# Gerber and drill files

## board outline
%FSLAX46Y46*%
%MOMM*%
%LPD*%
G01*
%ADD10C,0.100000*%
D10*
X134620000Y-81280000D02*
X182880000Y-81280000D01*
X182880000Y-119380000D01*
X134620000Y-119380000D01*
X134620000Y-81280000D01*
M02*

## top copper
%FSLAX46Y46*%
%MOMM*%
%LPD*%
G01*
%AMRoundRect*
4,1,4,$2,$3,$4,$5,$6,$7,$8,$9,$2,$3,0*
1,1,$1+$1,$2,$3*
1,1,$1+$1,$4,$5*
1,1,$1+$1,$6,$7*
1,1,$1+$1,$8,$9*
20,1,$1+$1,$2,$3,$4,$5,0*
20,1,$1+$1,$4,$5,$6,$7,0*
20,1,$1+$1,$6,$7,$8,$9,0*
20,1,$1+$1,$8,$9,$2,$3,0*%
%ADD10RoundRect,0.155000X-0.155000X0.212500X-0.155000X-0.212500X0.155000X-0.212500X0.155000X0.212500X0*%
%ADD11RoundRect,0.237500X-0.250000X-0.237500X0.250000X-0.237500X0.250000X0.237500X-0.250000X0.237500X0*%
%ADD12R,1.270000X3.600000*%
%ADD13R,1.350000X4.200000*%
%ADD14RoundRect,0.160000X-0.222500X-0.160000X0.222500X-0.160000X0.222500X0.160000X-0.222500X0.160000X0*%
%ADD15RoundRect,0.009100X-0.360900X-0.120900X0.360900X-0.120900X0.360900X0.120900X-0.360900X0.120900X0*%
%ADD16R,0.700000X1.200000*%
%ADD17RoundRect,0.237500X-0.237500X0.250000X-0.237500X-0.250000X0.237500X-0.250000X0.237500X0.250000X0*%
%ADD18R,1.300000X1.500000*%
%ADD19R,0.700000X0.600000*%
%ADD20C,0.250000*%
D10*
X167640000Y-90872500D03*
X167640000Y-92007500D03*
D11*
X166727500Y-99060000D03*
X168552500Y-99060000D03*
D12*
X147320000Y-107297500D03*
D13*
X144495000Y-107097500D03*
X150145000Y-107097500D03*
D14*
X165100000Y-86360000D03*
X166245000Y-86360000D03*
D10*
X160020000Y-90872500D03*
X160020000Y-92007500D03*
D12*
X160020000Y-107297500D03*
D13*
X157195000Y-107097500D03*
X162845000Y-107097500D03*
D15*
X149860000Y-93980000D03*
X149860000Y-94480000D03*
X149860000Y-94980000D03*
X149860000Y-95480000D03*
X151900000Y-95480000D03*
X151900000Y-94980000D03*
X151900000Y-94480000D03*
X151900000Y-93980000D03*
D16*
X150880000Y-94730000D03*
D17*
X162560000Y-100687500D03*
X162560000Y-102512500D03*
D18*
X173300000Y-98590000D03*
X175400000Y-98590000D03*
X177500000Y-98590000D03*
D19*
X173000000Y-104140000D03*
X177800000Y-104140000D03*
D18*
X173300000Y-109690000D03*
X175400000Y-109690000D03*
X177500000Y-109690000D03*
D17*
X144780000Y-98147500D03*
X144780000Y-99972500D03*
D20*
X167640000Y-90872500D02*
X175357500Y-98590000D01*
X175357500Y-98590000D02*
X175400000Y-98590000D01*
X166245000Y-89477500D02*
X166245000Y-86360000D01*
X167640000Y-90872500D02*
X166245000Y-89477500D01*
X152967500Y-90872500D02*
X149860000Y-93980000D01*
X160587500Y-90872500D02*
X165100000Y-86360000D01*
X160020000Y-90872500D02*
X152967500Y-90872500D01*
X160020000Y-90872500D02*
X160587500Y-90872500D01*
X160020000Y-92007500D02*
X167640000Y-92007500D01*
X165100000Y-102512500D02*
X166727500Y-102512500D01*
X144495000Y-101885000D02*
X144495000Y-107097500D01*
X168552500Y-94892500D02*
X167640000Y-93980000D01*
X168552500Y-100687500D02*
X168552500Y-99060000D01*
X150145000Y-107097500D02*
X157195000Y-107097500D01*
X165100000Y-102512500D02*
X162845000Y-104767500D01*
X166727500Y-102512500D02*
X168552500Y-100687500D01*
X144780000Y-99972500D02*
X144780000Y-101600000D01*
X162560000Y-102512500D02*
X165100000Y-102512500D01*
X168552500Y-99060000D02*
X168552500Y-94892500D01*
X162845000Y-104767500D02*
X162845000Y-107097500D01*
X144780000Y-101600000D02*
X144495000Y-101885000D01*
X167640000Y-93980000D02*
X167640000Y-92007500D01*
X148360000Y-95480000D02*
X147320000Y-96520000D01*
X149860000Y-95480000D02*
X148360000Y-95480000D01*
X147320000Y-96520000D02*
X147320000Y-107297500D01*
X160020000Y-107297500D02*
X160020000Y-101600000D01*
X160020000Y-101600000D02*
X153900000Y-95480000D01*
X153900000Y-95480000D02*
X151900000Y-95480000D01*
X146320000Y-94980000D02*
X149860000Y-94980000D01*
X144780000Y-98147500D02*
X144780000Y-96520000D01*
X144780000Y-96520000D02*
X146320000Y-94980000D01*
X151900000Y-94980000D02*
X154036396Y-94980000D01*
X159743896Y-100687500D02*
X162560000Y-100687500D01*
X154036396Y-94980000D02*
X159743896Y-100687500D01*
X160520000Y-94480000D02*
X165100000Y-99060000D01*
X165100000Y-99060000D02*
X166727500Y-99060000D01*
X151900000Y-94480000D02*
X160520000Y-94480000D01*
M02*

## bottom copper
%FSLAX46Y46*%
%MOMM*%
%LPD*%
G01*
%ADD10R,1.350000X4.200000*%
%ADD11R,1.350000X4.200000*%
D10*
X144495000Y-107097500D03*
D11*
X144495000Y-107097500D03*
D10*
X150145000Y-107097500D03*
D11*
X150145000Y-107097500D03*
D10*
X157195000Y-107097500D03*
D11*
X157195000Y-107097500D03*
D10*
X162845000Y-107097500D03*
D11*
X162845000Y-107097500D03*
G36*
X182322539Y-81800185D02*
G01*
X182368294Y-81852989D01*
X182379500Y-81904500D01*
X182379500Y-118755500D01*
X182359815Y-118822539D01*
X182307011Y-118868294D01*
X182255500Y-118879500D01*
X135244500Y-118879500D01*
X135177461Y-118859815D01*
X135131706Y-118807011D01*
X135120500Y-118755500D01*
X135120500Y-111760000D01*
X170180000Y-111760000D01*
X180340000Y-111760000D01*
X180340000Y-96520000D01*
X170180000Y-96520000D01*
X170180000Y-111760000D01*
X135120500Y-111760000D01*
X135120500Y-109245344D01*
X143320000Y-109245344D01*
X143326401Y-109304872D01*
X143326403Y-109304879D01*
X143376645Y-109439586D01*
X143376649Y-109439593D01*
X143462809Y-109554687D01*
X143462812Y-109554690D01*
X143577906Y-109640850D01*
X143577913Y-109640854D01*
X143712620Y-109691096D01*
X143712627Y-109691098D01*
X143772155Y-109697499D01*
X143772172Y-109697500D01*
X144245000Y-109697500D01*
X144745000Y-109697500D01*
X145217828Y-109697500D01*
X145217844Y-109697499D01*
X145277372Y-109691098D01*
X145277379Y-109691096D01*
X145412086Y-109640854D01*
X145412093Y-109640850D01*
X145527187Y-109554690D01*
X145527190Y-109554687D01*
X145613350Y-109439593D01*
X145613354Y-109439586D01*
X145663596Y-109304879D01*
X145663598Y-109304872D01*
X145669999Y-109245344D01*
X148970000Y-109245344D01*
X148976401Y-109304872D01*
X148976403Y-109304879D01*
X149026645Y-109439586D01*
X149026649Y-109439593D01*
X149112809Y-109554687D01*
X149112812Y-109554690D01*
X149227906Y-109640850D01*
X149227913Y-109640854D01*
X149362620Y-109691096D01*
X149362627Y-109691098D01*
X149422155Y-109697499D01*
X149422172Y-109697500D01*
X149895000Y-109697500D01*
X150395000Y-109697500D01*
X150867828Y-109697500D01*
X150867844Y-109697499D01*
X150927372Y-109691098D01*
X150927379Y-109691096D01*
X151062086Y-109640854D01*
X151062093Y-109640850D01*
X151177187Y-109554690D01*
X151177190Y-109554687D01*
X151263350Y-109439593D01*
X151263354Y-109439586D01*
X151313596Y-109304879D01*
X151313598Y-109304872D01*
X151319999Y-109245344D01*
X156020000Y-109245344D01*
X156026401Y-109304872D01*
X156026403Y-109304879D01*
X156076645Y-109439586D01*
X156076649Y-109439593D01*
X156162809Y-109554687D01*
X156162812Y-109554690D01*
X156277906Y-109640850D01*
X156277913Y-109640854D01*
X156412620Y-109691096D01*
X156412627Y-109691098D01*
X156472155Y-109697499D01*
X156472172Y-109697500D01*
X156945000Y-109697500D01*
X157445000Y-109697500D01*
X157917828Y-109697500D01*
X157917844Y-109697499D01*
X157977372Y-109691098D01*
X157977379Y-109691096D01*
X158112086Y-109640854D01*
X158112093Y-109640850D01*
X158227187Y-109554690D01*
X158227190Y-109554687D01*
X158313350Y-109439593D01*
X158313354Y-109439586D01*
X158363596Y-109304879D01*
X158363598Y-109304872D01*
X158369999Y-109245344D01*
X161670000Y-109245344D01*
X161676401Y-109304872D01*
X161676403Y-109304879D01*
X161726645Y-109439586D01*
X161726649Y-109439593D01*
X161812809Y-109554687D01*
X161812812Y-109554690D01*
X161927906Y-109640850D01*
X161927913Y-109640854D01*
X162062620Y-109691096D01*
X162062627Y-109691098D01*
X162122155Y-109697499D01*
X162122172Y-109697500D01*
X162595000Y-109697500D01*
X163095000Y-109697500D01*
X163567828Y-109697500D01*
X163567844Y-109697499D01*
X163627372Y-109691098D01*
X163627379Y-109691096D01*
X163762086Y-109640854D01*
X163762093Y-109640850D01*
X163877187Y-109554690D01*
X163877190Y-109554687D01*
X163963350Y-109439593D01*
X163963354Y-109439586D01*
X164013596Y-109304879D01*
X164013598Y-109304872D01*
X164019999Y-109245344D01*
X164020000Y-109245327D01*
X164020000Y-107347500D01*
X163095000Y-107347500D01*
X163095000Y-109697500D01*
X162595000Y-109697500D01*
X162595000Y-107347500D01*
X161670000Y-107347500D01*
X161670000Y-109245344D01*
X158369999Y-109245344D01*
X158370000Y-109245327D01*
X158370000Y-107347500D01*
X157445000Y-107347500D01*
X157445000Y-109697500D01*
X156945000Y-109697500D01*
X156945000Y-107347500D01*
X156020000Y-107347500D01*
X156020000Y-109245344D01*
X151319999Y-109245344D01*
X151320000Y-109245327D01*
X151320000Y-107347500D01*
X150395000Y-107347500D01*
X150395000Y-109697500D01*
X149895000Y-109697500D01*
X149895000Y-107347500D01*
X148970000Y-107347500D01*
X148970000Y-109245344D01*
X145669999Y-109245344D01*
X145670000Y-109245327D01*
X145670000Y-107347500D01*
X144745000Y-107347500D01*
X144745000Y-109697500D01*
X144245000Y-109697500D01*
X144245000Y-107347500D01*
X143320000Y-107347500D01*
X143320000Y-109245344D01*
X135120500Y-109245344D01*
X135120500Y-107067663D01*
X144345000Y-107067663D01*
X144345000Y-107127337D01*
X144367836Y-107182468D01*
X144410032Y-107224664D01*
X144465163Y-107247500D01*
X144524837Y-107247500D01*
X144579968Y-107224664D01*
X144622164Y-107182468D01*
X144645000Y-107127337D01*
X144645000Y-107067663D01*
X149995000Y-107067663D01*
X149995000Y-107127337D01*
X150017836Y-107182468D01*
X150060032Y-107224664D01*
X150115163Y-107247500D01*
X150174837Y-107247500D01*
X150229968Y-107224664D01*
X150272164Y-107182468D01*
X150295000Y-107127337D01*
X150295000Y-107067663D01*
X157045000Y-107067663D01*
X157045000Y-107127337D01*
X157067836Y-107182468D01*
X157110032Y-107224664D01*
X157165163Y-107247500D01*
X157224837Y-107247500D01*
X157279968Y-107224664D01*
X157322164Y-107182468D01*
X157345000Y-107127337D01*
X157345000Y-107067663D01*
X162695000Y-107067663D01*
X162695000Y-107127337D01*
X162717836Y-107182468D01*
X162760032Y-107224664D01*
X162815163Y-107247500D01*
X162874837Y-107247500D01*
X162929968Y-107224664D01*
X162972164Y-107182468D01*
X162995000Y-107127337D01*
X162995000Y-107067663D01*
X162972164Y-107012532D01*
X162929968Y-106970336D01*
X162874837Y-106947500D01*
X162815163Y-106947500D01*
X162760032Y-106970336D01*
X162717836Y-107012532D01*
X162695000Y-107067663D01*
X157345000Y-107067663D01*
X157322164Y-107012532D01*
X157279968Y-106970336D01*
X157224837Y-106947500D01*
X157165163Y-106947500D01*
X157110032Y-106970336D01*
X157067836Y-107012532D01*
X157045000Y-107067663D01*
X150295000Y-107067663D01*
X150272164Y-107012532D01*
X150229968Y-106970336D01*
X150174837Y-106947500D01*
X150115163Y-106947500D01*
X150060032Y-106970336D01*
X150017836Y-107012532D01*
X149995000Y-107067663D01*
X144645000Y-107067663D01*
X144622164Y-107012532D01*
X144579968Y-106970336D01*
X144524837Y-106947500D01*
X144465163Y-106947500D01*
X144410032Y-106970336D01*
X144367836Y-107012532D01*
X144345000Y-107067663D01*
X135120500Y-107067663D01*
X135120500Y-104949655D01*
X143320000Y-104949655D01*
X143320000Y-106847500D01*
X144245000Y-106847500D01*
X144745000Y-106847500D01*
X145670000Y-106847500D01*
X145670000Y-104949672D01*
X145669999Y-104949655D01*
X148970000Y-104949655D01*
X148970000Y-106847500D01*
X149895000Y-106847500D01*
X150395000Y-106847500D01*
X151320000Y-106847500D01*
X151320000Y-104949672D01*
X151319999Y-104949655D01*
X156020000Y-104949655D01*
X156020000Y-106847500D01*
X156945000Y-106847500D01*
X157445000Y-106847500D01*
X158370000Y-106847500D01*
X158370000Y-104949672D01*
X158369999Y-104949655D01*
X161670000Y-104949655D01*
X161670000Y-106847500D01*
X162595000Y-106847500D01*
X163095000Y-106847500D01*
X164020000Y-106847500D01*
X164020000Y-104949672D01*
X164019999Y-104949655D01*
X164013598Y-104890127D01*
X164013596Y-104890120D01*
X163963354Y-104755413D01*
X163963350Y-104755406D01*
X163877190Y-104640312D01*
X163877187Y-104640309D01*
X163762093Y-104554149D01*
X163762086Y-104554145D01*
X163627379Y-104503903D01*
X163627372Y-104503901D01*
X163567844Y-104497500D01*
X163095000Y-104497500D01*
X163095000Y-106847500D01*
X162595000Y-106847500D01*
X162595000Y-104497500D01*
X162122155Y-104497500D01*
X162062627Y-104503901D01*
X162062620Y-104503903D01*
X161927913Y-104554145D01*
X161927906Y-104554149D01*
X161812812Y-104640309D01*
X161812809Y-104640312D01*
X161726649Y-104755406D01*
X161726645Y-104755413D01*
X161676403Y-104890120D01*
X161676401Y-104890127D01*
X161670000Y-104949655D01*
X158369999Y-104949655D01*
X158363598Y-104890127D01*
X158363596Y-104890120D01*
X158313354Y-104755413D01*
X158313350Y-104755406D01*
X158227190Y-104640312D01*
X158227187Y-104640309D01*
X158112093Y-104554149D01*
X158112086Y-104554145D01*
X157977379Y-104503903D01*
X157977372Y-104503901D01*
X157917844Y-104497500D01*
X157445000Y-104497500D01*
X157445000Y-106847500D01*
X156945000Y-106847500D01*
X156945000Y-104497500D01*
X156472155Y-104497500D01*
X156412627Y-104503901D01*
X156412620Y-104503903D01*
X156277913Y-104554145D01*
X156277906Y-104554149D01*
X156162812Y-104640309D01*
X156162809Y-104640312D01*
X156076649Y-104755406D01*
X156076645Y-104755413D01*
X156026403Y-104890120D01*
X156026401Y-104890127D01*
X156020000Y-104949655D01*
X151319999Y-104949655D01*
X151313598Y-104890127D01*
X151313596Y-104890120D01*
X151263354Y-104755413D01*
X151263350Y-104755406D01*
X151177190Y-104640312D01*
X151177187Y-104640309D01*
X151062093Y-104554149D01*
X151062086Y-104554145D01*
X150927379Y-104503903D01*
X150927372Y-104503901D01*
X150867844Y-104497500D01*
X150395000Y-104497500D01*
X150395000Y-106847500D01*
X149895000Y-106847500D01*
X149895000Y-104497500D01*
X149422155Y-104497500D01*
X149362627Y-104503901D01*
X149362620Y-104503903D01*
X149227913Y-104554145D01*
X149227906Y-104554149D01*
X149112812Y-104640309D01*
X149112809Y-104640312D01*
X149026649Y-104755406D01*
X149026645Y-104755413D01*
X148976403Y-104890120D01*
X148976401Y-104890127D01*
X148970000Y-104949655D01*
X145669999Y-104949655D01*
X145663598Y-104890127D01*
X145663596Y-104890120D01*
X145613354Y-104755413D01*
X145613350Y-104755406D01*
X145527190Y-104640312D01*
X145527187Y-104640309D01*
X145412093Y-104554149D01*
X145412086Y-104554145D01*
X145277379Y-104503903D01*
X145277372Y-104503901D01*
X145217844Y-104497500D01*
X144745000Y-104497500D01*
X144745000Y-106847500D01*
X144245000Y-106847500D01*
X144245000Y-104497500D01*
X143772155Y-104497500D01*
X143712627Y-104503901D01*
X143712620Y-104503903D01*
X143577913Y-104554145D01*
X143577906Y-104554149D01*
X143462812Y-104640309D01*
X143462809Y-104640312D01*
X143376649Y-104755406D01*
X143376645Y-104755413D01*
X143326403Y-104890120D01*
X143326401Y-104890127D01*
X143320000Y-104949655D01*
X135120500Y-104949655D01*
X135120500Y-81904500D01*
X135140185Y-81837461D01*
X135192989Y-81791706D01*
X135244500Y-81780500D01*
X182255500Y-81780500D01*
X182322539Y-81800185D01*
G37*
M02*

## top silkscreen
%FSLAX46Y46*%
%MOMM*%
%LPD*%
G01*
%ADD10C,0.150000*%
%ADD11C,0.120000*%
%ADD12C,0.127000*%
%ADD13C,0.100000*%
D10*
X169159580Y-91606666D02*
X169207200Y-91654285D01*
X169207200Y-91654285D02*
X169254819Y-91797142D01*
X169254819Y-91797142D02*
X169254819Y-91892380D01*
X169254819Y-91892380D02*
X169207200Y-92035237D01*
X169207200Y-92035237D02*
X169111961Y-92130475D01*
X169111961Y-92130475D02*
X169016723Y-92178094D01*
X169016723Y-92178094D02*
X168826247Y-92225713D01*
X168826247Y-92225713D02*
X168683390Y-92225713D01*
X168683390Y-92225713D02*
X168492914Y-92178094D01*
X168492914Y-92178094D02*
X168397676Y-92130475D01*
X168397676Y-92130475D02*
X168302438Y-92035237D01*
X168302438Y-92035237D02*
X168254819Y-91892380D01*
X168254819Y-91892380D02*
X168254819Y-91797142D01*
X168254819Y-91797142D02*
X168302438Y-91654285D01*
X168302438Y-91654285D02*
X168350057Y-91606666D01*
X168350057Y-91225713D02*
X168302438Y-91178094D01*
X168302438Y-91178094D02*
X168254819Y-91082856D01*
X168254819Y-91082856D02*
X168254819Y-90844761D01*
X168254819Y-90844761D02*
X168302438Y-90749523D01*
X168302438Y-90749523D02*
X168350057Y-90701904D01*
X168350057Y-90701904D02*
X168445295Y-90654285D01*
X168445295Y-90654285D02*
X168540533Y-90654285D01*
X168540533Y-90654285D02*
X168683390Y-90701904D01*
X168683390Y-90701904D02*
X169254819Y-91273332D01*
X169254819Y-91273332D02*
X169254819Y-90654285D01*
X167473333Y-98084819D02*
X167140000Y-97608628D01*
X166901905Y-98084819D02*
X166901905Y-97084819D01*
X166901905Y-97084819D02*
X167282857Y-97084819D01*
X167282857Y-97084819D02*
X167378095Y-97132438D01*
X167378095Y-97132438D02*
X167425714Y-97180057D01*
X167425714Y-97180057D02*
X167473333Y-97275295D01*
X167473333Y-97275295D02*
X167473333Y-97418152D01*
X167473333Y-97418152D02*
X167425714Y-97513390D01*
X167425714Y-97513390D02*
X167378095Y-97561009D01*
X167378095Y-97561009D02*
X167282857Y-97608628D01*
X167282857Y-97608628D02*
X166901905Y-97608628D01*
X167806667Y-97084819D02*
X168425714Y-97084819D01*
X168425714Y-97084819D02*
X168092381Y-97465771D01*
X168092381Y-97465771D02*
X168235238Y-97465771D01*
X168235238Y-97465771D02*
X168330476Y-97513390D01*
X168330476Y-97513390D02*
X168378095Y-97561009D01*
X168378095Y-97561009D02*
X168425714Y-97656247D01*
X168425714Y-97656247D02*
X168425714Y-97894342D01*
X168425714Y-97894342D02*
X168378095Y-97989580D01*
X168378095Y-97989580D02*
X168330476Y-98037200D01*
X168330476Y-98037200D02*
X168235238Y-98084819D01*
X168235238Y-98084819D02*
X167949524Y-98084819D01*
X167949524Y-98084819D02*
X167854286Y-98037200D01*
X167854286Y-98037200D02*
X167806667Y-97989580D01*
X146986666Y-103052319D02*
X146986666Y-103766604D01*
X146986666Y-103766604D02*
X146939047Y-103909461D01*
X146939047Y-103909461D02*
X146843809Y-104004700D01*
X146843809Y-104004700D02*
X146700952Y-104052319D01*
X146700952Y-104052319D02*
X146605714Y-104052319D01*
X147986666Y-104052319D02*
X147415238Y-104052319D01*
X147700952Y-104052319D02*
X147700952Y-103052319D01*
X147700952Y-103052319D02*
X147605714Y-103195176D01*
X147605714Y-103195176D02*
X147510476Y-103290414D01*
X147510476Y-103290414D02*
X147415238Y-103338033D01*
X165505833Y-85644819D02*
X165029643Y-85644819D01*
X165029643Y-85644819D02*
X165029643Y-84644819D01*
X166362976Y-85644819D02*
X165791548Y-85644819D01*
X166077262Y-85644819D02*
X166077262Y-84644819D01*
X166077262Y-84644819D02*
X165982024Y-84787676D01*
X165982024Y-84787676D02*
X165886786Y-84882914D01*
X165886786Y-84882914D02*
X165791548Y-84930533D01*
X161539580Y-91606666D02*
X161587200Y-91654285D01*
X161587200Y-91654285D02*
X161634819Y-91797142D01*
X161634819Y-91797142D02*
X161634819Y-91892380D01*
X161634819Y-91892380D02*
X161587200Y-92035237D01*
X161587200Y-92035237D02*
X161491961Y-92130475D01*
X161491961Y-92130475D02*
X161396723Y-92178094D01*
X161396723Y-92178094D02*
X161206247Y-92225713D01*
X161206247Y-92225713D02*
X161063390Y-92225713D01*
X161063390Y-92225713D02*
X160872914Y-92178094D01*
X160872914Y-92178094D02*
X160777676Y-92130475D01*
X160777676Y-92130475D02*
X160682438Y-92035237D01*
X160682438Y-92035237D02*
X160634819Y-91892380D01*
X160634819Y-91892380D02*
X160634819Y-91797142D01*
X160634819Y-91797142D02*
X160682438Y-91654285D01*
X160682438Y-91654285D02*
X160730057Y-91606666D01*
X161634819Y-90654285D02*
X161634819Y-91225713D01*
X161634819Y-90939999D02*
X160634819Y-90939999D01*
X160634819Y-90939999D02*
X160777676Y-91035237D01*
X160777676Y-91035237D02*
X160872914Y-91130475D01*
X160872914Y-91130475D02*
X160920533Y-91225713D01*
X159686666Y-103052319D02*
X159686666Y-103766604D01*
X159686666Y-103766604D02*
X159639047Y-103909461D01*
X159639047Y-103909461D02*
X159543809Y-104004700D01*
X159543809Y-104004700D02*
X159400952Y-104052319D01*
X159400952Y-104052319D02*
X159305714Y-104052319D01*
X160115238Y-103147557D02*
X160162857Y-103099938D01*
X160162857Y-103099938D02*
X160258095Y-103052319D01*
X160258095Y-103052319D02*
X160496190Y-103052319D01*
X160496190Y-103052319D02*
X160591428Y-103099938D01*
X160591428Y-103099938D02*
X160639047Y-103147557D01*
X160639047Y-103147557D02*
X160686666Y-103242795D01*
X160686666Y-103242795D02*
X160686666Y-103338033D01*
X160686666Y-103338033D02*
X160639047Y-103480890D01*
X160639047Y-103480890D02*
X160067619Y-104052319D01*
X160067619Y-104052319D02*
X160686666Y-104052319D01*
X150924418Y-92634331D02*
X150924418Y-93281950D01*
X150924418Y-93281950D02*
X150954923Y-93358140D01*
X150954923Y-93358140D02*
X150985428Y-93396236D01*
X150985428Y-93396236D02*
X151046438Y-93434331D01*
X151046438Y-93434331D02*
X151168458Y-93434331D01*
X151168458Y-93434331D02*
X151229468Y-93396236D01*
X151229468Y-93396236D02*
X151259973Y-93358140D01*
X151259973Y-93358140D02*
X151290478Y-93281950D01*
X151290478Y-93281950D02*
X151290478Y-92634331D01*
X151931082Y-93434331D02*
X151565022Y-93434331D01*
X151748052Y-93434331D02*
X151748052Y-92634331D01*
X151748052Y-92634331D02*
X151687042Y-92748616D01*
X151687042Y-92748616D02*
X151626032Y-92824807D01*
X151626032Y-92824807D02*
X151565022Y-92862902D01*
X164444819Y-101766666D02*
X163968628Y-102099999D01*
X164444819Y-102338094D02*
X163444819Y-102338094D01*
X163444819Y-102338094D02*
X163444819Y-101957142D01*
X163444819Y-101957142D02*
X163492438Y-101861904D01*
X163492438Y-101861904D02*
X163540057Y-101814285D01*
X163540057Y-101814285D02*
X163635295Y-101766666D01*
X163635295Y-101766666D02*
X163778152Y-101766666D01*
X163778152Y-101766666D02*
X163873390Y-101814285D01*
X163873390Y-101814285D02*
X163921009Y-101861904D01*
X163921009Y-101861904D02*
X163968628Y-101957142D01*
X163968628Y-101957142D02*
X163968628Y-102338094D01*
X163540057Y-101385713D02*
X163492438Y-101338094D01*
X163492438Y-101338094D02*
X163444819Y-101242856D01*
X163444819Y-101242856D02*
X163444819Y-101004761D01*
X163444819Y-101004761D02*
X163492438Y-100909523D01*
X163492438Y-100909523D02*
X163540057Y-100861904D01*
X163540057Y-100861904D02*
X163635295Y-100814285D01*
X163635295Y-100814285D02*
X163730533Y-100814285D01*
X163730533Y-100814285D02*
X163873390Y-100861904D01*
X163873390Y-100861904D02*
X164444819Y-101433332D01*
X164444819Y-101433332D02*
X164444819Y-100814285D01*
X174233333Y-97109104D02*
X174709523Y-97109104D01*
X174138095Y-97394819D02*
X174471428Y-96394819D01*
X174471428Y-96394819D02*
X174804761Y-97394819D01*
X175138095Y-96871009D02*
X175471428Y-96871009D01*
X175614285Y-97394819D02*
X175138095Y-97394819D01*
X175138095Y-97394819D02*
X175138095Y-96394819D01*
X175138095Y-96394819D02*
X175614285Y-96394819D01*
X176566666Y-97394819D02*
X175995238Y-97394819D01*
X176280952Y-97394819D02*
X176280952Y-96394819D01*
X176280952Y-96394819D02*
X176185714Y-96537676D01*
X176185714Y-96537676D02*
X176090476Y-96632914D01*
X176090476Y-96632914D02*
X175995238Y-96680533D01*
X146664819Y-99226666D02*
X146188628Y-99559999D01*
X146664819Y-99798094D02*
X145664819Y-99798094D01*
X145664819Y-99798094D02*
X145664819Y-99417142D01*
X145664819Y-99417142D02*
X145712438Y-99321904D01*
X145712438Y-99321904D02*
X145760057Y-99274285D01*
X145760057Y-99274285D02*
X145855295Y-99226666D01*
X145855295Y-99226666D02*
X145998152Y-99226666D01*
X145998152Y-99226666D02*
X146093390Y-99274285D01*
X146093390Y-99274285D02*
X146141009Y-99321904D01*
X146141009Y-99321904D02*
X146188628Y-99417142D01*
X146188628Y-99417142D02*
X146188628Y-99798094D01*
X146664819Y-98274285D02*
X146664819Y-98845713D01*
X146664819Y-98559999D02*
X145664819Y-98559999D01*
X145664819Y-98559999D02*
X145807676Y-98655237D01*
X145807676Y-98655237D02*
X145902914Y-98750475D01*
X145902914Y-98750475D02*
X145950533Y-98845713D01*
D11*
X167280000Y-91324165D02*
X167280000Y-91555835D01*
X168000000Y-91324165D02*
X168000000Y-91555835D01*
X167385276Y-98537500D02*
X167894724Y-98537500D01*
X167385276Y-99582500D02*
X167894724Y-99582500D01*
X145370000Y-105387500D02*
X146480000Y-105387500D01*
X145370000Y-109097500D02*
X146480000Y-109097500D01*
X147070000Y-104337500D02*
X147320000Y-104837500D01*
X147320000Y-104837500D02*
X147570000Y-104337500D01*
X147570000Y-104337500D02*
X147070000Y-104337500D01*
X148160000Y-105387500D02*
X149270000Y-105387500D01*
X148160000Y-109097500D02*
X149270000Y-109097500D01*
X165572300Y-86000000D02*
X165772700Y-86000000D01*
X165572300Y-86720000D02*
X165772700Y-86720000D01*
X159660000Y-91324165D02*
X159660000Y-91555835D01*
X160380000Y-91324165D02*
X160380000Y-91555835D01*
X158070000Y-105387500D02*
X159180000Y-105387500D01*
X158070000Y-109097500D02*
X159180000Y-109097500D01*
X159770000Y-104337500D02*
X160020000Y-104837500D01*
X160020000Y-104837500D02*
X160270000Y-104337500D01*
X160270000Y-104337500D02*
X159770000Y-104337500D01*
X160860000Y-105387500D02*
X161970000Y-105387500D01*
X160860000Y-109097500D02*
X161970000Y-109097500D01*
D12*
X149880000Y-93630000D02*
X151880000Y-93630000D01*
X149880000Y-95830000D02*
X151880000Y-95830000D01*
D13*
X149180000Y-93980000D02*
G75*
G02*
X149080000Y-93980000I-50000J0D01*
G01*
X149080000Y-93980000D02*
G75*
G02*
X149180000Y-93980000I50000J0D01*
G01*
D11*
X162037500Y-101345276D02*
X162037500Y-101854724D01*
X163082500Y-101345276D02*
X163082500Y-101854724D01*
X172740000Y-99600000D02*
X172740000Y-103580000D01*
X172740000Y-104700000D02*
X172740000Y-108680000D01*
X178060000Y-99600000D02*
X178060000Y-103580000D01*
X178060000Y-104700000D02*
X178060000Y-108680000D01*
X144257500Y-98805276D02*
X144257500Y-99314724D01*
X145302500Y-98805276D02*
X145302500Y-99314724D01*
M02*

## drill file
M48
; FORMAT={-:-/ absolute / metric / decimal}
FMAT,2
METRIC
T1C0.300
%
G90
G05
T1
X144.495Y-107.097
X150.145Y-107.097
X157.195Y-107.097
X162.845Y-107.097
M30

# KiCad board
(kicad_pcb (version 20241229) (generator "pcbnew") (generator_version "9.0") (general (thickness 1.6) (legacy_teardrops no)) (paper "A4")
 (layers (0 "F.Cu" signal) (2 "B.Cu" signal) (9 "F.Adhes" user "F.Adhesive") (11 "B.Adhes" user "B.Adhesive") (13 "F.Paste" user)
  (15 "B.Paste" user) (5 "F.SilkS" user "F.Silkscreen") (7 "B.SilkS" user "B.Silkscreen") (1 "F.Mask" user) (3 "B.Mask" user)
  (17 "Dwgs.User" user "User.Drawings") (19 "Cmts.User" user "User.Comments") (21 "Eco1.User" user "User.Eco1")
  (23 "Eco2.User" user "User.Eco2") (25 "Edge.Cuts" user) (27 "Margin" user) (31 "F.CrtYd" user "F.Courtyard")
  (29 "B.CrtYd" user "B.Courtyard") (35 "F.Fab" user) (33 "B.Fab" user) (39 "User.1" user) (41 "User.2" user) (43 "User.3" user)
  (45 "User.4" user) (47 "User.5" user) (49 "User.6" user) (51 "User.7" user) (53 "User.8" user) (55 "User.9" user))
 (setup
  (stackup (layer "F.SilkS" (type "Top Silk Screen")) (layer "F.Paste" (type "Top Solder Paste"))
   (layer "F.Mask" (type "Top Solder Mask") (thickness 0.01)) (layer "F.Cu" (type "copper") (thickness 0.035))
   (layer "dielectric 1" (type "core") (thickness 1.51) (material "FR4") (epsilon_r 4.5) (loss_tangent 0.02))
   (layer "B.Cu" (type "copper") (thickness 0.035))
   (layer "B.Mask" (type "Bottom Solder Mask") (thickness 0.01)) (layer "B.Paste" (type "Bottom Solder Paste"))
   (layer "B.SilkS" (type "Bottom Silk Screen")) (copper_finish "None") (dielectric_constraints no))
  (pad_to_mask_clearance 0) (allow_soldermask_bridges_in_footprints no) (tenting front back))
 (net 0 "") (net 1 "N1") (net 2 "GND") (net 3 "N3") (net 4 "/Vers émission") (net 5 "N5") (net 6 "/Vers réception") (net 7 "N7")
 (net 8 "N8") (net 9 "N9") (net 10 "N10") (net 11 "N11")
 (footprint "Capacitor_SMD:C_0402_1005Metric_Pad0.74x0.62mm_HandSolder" (layer "F.Cu") (at 167.64 91.44 -90)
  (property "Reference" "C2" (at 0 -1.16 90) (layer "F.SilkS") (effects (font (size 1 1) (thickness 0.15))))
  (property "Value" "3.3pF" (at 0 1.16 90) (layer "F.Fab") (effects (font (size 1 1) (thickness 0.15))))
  (fp_line (start -0.115835 0.36) (end 0.115835 0.36) (stroke (width 0.12) (type solid)) (layer "F.SilkS"))
  (fp_line (start -0.115835 -0.36) (end 0.115835 -0.36) (stroke (width 0.12) (type solid)) (layer "F.SilkS"))
  (pad "1" smd roundrect (at -0.5675 0 270) (size 0.735 0.62) (layers "F.Cu" "F.Mask" "F.Paste") (roundrect_rratio 0.25) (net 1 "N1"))
  (pad "2" smd roundrect (at 0.5675 0 270) (size 0.735 0.62) (layers "F.Cu" "F.Mask" "F.Paste") (roundrect_rratio 0.25) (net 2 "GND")))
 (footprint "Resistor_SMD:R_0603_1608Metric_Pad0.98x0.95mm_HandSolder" (layer "F.Cu") (at 167.64 99.06)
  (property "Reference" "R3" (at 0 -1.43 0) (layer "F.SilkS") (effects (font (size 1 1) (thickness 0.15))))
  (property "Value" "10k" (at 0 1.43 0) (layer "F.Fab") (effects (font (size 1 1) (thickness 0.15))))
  (fp_line (start -0.254724 -0.5225) (end 0.254724 -0.5225) (stroke (width 0.12) (type solid)) (layer "F.SilkS"))
  (fp_line (start -0.254724 0.5225) (end 0.254724 0.5225) (stroke (width 0.12) (type solid)) (layer "F.SilkS"))
  (pad "1" smd roundrect (at -0.9125 0) (size 0.975 0.95) (layers "F.Cu" "F.Mask" "F.Paste") (roundrect_rratio 0.25) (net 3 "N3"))
  (pad "2" smd roundrect (at 0.9125 0) (size 0.975 0.95) (layers "F.Cu" "F.Mask" "F.Paste") (roundrect_rratio 0.25) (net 2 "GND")))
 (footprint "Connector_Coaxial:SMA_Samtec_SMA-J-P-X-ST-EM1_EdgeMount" (layer "F.Cu") (at 147.32 107.0975)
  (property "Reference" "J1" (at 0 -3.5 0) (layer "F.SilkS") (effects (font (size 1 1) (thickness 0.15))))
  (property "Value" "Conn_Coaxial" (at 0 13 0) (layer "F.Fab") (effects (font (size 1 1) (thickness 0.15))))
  (fp_line (start -1.95 -1.71) (end -0.84 -1.71) (stroke (width 0.12) (type solid)) (layer "F.SilkS"))
  (fp_line (start -1.95 2) (end -0.84 2) (stroke (width 0.12) (type solid)) (layer "F.SilkS"))
  (fp_line (start -0.25 -2.76) (end 0 -2.26) (stroke (width 0.12) (type solid)) (layer "F.SilkS"))
  (fp_line (start 0 -2.26) (end 0.25 -2.76) (stroke (width 0.12) (type solid)) (layer "F.SilkS"))
  (fp_line (start 0.25 -2.76) (end -0.25 -2.76) (stroke (width 0.12) (type solid)) (layer "F.SilkS"))
  (fp_line (start 0.84 -1.71) (end 1.95 -1.71) (stroke (width 0.12) (type solid)) (layer "F.SilkS"))
  (fp_line (start 0.84 2) (end 1.95 2) (stroke (width 0.12) (type solid)) (layer "F.SilkS"))
  (pad "1" smd rect (at 0 0.2) (size 1.27 3.6) (layers "F.Cu" "F.Mask" "F.Paste") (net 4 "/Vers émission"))
  (pad "2" thru_hole rect (at -2.825 0) (size 1.35 4.2) (drill 0.3) (layers "*.Cu" "*.Mask") (remove_unused_layers no) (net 2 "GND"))
  (pad "2" smd rect (at -2.825 0) (size 1.35 4.2) (layers "B.Cu" "B.Mask" "B.Paste") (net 2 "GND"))
  (pad "2" thru_hole rect (at 2.825 0) (size 1.35 4.2) (drill 0.3) (layers "*.Cu" "*.Mask") (remove_unused_layers no) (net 2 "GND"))
  (pad "2" smd rect (at 2.825 0) (size 1.35 4.2) (layers "B.Cu" "B.Mask" "B.Paste") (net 2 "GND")))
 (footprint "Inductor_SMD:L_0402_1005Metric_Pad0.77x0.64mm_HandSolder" (layer "F.Cu") (at 165.6725 86.36)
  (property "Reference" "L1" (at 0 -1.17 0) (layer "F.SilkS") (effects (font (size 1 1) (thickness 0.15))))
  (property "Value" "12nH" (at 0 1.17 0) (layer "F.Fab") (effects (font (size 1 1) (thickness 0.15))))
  (fp_line (start -0.1002 -0.36) (end 0.1002 -0.36) (stroke (width 0.12) (type solid)) (layer "F.SilkS"))
  (fp_line (start -0.1002 0.36) (end 0.1002 0.36) (stroke (width 0.12) (type solid)) (layer "F.SilkS"))
  (pad "1" smd roundrect (at -0.5725 0) (size 0.765 0.64) (layers "F.Cu" "F.Mask" "F.Paste") (roundrect_rratio 0.25) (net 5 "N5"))
  (pad "2" smd roundrect (at 0.5725 0) (size 0.765 0.64) (layers "F.Cu" "F.Mask" "F.Paste") (roundrect_rratio 0.25) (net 1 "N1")))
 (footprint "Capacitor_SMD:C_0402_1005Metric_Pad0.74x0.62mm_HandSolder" (layer "F.Cu") (at 160.02 91.44 -90)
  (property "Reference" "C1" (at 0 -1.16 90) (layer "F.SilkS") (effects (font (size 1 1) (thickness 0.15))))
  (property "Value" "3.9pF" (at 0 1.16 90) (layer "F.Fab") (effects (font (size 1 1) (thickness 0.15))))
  (fp_line (start -0.115835 0.36) (end 0.115835 0.36) (stroke (width 0.12) (type solid)) (layer "F.SilkS"))
  (fp_line (start -0.115835 -0.36) (end 0.115835 -0.36) (stroke (width 0.12) (type solid)) (layer "F.SilkS"))
  (pad "1" smd roundrect (at -0.5675 0 270) (size 0.735 0.62) (layers "F.Cu" "F.Mask" "F.Paste") (roundrect_rratio 0.25) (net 5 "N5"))
  (pad "2" smd roundrect (at 0.5675 0 270) (size 0.735 0.62) (layers "F.Cu" "F.Mask" "F.Paste") (roundrect_rratio 0.25) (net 2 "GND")))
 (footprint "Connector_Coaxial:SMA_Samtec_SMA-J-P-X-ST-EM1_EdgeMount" (layer "F.Cu") (at 160.02 107.0975)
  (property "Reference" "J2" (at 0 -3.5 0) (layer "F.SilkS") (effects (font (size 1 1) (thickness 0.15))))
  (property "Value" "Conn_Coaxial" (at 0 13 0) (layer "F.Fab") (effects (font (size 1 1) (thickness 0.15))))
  (fp_line (start -1.95 -1.71) (end -0.84 -1.71) (stroke (width 0.12) (type solid)) (layer "F.SilkS"))
  (fp_line (start -1.95 2) (end -0.84 2) (stroke (width 0.12) (type solid)) (layer "F.SilkS"))
  (fp_line (start -0.25 -2.76) (end 0 -2.26) (stroke (width 0.12) (type solid)) (layer "F.SilkS"))
  (fp_line (start 0 -2.26) (end 0.25 -2.76) (stroke (width 0.12) (type solid)) (layer "F.SilkS"))
  (fp_line (start 0.25 -2.76) (end -0.25 -2.76) (stroke (width 0.12) (type solid)) (layer "F.SilkS"))
  (fp_line (start 0.84 -1.71) (end 1.95 -1.71) (stroke (width 0.12) (type solid)) (layer "F.SilkS"))
  (fp_line (start 0.84 2) (end 1.95 2) (stroke (width 0.12) (type solid)) (layer "F.SilkS"))
  (pad "1" smd rect (at 0 0.2) (size 1.27 3.6) (layers "F.Cu" "F.Mask" "F.Paste") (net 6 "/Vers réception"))
  (pad "2" thru_hole rect (at -2.825 0) (size 1.35 4.2) (drill 0.3) (layers "*.Cu" "*.Mask") (remove_unused_layers no) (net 2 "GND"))
  (pad "2" smd rect (at -2.825 0) (size 1.35 4.2) (layers "B.Cu" "B.Mask" "B.Paste") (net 2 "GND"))
  (pad "2" thru_hole rect (at 2.825 0) (size 1.35 4.2) (drill 0.3) (layers "*.Cu" "*.Mask") (remove_unused_layers no) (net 2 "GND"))
  (pad "2" smd rect (at 2.825 0) (size 1.35 4.2) (layers "B.Cu" "B.Mask" "B.Paste") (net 2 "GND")))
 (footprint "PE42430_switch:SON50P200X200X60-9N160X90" (layer "F.Cu") (at 150.88 94.73)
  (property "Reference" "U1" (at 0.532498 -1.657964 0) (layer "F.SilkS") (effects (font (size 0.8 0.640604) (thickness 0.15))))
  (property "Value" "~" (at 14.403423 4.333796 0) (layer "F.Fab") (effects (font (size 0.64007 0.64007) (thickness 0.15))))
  (fp_line (start -1 -1.1) (end 1 -1.1) (stroke (width 0.127) (type solid)) (layer "F.SilkS"))
  (fp_line (start -1 1.1) (end 1 1.1) (stroke (width 0.127) (type solid)) (layer "F.SilkS"))
  (fp_circle (center -1.75 -0.75) (end -1.7 -0.75) (stroke (width 0.1) (type solid)) (fill no) (layer "F.SilkS"))
  (pad "1" smd roundrect (at -1.02 -0.75) (size 0.74 0.26) (layers "F.Cu" "F.Mask" "F.Paste") (roundrect_rratio 0.035) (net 5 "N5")
   (solder_mask_margin 0.102))
  (pad "2" smd roundrect (at -1.02 -0.25) (size 0.74 0.26) (layers "F.Cu" "F.Mask" "F.Paste") (roundrect_rratio 0.035) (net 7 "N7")
   (solder_mask_margin 0.102))
  (pad "3" smd roundrect (at -1.02 0.25) (size 0.74 0.26) (layers "F.Cu" "F.Mask" "F.Paste") (roundrect_rratio 0.035) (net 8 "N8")
   (solder_mask_margin 0.102))
  (pad "4" smd roundrect (at -1.02 0.75) (size 0.74 0.26) (layers "F.Cu" "F.Mask" "F.Paste") (roundrect_rratio 0.035)
   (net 4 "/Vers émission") (solder_mask_margin 0.102))
  (pad "5" smd roundrect (at 1.02 0.75) (size 0.74 0.26) (layers "F.Cu" "F.Mask" "F.Paste") (roundrect_rratio 0.035)
   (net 6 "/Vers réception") (solder_mask_margin 0.102))
  (pad "6" smd roundrect (at 1.02 0.25) (size 0.74 0.26) (layers "F.Cu" "F.Mask" "F.Paste") (roundrect_rratio 0.035) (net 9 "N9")
   (solder_mask_margin 0.102))
  (pad "7" smd roundrect (at 1.02 -0.25) (size 0.74 0.26) (layers "F.Cu" "F.Mask" "F.Paste") (roundrect_rratio 0.035) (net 3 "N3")
   (solder_mask_margin 0.102))
  (pad "8" smd roundrect (at 1.02 -0.75) (size 0.74 0.26) (layers "F.Cu" "F.Mask" "F.Paste") (roundrect_rratio 0.035) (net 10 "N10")
   (solder_mask_margin 0.102))
  (pad "EP" smd rect (at 0 0) (size 0.7 1.2) (layers "F.Cu" "F.Mask") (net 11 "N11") (solder_mask_margin 0.102)))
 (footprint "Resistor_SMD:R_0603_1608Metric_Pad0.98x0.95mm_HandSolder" (layer "F.Cu") (at 162.56 101.6 -90)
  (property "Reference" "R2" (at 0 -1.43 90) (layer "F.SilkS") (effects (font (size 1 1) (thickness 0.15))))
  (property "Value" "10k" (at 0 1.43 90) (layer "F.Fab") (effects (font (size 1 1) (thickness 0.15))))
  (fp_line (start -0.254724 0.5225) (end 0.254724 0.5225) (stroke (width 0.12) (type solid)) (layer "F.SilkS"))
  (fp_line (start -0.254724 -0.5225) (end 0.254724 -0.5225) (stroke (width 0.12) (type solid)) (layer "F.SilkS"))
  (pad "1" smd roundrect (at -0.9125 0 270) (size 0.975 0.95) (layers "F.Cu" "F.Mask" "F.Paste") (roundrect_rratio 0.25) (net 9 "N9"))
  (pad "2" smd roundrect (at 0.9125 0 270) (size 0.975 0.95) (layers "F.Cu" "F.Mask" "F.Paste") (roundrect_rratio 0.25) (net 2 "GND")))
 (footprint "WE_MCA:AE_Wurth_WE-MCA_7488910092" (layer "F.Cu") (at 175.4 104.14)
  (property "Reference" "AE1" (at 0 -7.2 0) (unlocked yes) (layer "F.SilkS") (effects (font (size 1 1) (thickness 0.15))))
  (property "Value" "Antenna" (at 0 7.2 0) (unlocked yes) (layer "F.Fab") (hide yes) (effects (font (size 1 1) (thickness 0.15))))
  (fp_line (start -2.66 -4.54) (end -2.66 -0.56) (stroke (width 0.12) (type default)) (layer "F.SilkS"))
  (fp_line (start -2.66 0.56) (end -2.66 4.54) (stroke (width 0.12) (type default)) (layer "F.SilkS"))
  (fp_line (start 2.66 -4.54) (end 2.66 -0.56) (stroke (width 0.12) (type default)) (layer "F.SilkS"))
  (fp_line (start 2.66 0.56) (end 2.66 4.54) (stroke (width 0.12) (type default)) (layer "F.SilkS"))
  (pad "1" smd rect (at -2.1 -5.55) (size 1.3 1.5) (layers "F.Cu" "F.Mask" "F.Paste"))
  (pad "2" smd rect (at 0 -5.55) (size 1.3 1.5) (layers "F.Cu" "F.Mask" "F.Paste") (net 1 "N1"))
  (pad "3" smd rect (at 2.1 -5.55) (size 1.3 1.5) (layers "F.Cu" "F.Mask" "F.Paste"))
  (pad "4" smd rect (at -2.4 0) (size 0.7 0.6) (layers "F.Cu" "F.Mask" "F.Paste"))
  (pad "5" smd rect (at 2.4 0) (size 0.7 0.6) (layers "F.Cu" "F.Mask" "F.Paste"))
  (pad "6" smd rect (at -2.1 5.55) (size 1.3 1.5) (layers "F.Cu" "F.Mask" "F.Paste"))
  (pad "7" smd rect (at 0 5.55) (size 1.3 1.5) (layers "F.Cu" "F.Mask" "F.Paste"))
  (pad "8" smd rect (at 2.1 5.55) (size 1.3 1.5) (layers "F.Cu" "F.Mask" "F.Paste")))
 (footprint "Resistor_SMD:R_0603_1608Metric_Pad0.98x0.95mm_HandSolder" (layer "F.Cu") (at 144.78 99.06 -90)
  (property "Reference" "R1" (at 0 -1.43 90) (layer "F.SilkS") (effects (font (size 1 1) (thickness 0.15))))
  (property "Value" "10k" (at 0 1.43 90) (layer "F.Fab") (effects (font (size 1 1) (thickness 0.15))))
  (fp_line (start -0.254724 0.5225) (end 0.254724 0.5225) (stroke (width 0.12) (type solid)) (layer "F.SilkS"))
  (fp_line (start -0.254724 -0.5225) (end 0.254724 -0.5225) (stroke (width 0.12) (type solid)) (layer "F.SilkS"))
  (pad "1" smd roundrect (at -0.9125 0 270) (size 0.975 0.95) (layers "F.Cu" "F.Mask" "F.Paste") (roundrect_rratio 0.25) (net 8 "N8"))
  (pad "2" smd roundrect (at 0.9125 0 270) (size 0.975 0.95) (layers "F.Cu" "F.Mask" "F.Paste") (roundrect_rratio 0.25) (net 2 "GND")))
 (gr_rect (start 134.62 81.28) (end 182.88 119.38) (stroke (width 0.1) (type default)) (fill no) (layer "Edge.Cuts"))
 (segment (start 167.64 90.8725) (end 175.3575 98.59) (width 0.25) (layer "F.Cu") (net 1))
 (segment (start 175.3575 98.59) (end 175.4 98.59) (width 0.25) (layer "F.Cu") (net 1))
 (segment (start 166.245 89.4775) (end 166.245 86.36) (width 0.25) (layer "F.Cu") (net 1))
 (segment (start 167.64 90.8725) (end 166.245 89.4775) (width 0.25) (layer "F.Cu") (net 1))
 (segment (start 152.9675 90.8725) (end 149.86 93.98) (width 0.25) (layer "F.Cu") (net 5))
 (segment (start 160.5875 90.8725) (end 165.1 86.36) (width 0.25) (layer "F.Cu") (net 5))
 (segment (start 160.02 90.8725) (end 152.9675 90.8725) (width 0.25) (layer "F.Cu") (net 5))
 (segment (start 160.02 90.8725) (end 160.5875 90.8725) (width 0.25) (layer "F.Cu") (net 5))
 (segment (start 160.02 92.0075) (end 167.64 92.0075) (width 0.25) (layer "F.Cu") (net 2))
 (segment (start 165.1 102.5125) (end 166.7275 102.5125) (width 0.25) (layer "F.Cu") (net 2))
 (segment (start 144.495 101.885) (end 144.495 107.0975) (width 0.25) (layer "F.Cu") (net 2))
 (segment (start 168.5525 94.8925) (end 167.64 93.98) (width 0.25) (layer "F.Cu") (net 2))
 (segment (start 168.5525 100.6875) (end 168.5525 99.06) (width 0.25) (layer "F.Cu") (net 2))
 (segment (start 150.145 107.0975) (end 157.195 107.0975) (width 0.25) (layer "F.Cu") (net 2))
 (segment (start 165.1 102.5125) (end 162.845 104.7675) (width 0.25) (layer "F.Cu") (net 2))
 (segment (start 166.7275 102.5125) (end 168.5525 100.6875) (width 0.25) (layer "F.Cu") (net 2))
 (segment (start 144.78 99.9725) (end 144.78 101.6) (width 0.25) (layer "F.Cu") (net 2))
 (segment (start 162.56 102.5125) (end 165.1 102.5125) (width 0.25) (layer "F.Cu") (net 2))
 (segment (start 168.5525 99.06) (end 168.5525 94.8925) (width 0.25) (layer "F.Cu") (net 2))
 (segment (start 162.845 104.7675) (end 162.845 107.0975) (width 0.25) (layer "F.Cu") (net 2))
 (segment (start 144.78 101.6) (end 144.495 101.885) (width 0.25) (layer "F.Cu") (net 2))
 (segment (start 167.64 93.98) (end 167.64 92.0075) (width 0.25) (layer "F.Cu") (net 2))
 (segment (start 148.36 95.48) (end 147.32 96.52) (width 0.25) (layer "F.Cu") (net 4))
 (segment (start 149.86 95.48) (end 148.36 95.48) (width 0.25) (layer "F.Cu") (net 4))
 (segment (start 147.32 96.52) (end 147.32 107.2975) (width 0.25) (layer "F.Cu") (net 4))
 (segment (start 160.02 107.2975) (end 160.02 101.6) (width 0.25) (layer "F.Cu") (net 6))
 (segment (start 160.02 101.6) (end 153.9 95.48) (width 0.25) (layer "F.Cu") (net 6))
 (segment (start 153.9 95.48) (end 151.9 95.48) (width 0.25) (layer "F.Cu") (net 6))
 (segment (start 146.32 94.98) (end 149.86 94.98) (width 0.25) (layer "F.Cu") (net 8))
 (segment (start 144.78 98.1475) (end 144.78 96.52) (width 0.25) (layer "F.Cu") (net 8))
 (segment (start 144.78 96.52) (end 146.32 94.98) (width 0.25) (layer "F.Cu") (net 8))
 (segment (start 151.9 94.98) (end 154.036396 94.98) (width 0.25) (layer "F.Cu") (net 9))
 (segment (start 159.743896 100.6875) (end 162.56 100.6875) (width 0.25) (layer "F.Cu") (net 9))
 (segment (start 154.036396 94.98) (end 159.743896 100.6875) (width 0.25) (layer "F.Cu") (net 9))
 (segment (start 160.52 94.48) (end 165.1 99.06) (width 0.25) (layer "F.Cu") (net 3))
 (segment (start 165.1 99.06) (end 166.7275 99.06) (width 0.25) (layer "F.Cu") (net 3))
 (segment (start 151.9 94.48) (end 160.52 94.48) (width 0.25) (layer "F.Cu") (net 3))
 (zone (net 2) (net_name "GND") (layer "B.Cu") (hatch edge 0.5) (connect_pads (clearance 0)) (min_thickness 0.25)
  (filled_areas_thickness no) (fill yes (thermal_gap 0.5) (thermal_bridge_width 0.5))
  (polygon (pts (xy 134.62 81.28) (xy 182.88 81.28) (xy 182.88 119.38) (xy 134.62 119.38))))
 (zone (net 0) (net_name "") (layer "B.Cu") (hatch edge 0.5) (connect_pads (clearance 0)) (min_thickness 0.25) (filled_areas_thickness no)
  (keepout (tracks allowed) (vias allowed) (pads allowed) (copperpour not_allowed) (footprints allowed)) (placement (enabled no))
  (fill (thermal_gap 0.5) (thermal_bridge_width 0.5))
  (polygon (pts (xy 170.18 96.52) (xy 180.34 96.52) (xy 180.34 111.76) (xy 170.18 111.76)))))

